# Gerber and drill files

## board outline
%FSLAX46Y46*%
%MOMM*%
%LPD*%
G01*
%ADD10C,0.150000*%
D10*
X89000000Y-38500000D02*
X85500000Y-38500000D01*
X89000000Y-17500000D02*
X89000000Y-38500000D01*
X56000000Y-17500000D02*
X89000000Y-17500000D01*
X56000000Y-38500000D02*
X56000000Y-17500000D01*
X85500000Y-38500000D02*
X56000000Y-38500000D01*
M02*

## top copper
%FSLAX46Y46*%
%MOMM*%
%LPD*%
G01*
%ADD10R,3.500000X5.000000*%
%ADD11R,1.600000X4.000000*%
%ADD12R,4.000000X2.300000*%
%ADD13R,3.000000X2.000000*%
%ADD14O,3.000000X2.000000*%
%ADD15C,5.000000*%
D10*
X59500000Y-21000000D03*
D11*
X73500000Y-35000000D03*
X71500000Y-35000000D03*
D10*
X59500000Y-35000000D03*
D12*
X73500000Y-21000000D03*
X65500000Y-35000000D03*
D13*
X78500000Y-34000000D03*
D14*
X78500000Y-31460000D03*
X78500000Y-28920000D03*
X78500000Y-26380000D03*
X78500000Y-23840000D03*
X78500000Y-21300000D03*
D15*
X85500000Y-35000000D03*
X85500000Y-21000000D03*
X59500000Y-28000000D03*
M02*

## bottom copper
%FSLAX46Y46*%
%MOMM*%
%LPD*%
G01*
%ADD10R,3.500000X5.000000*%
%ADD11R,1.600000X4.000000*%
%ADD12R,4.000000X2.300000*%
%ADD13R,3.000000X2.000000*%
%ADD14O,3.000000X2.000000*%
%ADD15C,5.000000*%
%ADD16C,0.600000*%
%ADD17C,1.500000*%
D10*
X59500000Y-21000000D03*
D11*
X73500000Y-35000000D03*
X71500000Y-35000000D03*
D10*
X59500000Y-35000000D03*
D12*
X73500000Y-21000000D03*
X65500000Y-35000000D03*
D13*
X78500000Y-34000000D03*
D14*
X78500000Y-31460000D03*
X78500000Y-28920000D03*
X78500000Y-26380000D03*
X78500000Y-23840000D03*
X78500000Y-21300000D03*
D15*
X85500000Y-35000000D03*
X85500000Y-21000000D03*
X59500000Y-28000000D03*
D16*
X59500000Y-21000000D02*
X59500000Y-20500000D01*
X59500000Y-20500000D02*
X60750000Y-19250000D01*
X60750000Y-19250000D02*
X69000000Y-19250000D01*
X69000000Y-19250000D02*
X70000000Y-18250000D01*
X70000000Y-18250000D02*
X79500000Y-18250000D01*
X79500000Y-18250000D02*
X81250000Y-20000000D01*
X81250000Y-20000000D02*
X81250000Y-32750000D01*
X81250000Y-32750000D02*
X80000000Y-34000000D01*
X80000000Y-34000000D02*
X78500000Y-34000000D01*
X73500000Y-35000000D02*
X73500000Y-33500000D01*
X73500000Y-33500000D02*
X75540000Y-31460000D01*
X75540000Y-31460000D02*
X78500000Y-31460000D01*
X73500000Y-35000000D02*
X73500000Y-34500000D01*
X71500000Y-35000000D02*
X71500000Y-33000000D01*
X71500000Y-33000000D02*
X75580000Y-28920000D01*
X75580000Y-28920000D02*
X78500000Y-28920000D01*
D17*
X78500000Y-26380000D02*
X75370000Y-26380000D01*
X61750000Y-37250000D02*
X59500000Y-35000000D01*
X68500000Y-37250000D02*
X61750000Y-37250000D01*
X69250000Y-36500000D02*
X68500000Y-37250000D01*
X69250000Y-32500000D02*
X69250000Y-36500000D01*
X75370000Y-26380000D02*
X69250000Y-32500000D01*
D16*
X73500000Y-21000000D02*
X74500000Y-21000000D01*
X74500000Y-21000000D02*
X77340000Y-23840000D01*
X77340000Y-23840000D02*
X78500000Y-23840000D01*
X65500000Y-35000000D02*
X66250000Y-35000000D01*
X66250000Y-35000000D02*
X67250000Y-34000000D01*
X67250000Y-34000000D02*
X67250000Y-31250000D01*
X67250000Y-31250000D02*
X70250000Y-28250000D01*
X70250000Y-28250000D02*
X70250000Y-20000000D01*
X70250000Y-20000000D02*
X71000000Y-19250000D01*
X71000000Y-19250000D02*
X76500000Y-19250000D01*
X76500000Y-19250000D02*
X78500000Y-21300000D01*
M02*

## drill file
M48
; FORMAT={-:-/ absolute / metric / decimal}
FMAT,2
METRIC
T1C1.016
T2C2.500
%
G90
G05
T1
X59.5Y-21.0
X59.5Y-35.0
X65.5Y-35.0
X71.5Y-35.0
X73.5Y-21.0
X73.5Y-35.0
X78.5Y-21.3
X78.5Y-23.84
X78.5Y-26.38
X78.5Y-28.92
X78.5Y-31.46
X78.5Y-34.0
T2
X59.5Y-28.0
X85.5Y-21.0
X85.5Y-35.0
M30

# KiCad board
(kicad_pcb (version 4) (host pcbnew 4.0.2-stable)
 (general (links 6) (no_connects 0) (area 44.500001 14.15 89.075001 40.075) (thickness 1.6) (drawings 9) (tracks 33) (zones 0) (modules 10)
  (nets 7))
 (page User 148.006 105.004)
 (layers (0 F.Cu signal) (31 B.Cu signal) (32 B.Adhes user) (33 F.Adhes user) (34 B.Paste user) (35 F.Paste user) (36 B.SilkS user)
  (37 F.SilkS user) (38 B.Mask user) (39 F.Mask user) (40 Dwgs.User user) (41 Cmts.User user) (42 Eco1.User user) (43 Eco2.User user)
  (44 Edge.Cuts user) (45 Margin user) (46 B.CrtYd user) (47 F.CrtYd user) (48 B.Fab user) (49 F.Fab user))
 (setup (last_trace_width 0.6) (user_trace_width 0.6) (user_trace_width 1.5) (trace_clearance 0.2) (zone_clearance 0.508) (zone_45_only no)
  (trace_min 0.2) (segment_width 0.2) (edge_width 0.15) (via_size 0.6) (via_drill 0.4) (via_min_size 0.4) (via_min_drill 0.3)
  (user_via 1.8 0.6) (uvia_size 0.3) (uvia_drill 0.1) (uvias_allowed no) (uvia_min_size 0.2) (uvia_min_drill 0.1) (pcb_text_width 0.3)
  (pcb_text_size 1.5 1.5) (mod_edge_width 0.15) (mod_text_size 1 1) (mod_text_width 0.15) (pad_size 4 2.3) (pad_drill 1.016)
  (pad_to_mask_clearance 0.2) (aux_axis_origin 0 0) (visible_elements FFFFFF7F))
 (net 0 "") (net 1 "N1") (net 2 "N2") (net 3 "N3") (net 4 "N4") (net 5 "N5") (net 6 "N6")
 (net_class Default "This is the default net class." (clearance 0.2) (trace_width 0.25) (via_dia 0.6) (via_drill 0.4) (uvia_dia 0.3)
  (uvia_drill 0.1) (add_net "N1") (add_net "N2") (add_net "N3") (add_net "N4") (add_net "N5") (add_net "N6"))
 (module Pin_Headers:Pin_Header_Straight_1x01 (layer F.Cu) (at 59.5 21)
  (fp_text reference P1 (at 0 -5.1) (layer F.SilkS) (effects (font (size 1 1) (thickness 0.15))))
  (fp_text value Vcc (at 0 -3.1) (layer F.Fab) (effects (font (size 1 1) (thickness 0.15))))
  (pad 1 thru_hole rect (at 0 0) (size 3.5 5) (drill 1.016) (layers *.Cu *.Mask F.SilkS) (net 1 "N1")))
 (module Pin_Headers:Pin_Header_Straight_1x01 (layer F.Cu) (at 73.5 35)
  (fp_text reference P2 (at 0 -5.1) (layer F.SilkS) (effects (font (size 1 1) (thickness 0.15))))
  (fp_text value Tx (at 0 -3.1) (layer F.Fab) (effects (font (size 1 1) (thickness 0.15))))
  (pad 1 thru_hole rect (at 0 0) (size 1.6 4) (drill 1.016) (layers *.Cu *.Mask F.SilkS) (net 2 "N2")))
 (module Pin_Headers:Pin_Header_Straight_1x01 (layer F.Cu) (at 71.5 35)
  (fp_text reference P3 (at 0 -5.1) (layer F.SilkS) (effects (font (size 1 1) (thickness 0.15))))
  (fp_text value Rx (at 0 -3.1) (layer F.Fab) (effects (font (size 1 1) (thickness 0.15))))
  (pad 1 thru_hole rect (at 0 0) (size 1.6 4) (drill 1.016) (layers *.Cu *.Mask F.SilkS) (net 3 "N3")))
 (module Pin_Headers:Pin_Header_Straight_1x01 (layer F.Cu) (at 59.5 35)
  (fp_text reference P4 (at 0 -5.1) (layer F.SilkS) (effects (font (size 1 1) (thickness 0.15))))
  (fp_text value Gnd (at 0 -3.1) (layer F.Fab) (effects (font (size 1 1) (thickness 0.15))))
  (pad 1 thru_hole rect (at 0 0) (size 3.5 5) (drill 1.016) (layers *.Cu *.Mask F.SilkS) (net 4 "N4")))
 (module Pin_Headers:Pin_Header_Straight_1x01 (layer F.Cu) (at 73.5 21)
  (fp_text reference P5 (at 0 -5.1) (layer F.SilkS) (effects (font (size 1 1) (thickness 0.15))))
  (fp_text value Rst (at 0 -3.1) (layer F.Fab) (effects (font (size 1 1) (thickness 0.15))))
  (pad 1 thru_hole rect (at 0 0) (size 4 2.3) (drill 1.016) (layers *.Cu *.Mask F.SilkS) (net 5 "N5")))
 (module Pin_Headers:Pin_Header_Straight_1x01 (layer F.Cu) (at 65.5 35)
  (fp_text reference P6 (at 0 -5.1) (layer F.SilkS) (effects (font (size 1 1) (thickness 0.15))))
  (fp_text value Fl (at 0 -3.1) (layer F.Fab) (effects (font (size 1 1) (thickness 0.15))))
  (pad 1 thru_hole rect (at 0 0) (size 4 2.3) (drill 1.016) (layers *.Cu *.Mask F.SilkS) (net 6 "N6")))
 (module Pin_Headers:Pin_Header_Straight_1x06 (layer F.Cu) (at 78.5 34 180)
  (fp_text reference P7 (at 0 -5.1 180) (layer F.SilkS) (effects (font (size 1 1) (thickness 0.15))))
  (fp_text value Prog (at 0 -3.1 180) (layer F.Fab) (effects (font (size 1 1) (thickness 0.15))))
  (pad 1 thru_hole rect (at 0 0 180) (size 3 2) (drill 1.016) (layers *.Cu *.Mask F.SilkS) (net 1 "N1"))
  (pad 2 thru_hole oval (at 0 2.54 180) (size 3 2) (drill 1.016) (layers *.Cu *.Mask F.SilkS) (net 2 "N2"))
  (pad 3 thru_hole oval (at 0 5.08 180) (size 3 2) (drill 1.016) (layers *.Cu *.Mask F.SilkS) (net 3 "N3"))
  (pad 4 thru_hole oval (at 0 7.62 180) (size 3 2) (drill 1.016) (layers *.Cu *.Mask F.SilkS) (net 4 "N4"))
  (pad 5 thru_hole oval (at 0 10.16 180) (size 3 2) (drill 1.016) (layers *.Cu *.Mask F.SilkS) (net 5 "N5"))
  (pad 6 thru_hole oval (at 0 12.7 180) (size 3 2) (drill 1.016) (layers *.Cu *.Mask F.SilkS) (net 6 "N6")))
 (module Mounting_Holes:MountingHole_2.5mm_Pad (layer F.Cu) (at 85.5 35)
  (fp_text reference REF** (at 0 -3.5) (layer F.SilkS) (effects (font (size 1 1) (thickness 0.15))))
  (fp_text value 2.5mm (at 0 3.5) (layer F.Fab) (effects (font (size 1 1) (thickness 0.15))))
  (pad 1 thru_hole circle (at 0 0) (size 5 5) (drill 2.5) (layers *.Cu *.Mask F.SilkS)))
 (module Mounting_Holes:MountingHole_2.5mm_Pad (layer F.Cu) (at 85.5 21)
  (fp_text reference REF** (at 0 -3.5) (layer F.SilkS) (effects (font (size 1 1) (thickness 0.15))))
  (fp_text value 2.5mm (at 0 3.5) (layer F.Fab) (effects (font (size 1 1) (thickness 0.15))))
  (pad 1 thru_hole circle (at 0 0) (size 5 5) (drill 2.5) (layers *.Cu *.Mask F.SilkS)))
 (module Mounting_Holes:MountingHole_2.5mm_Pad (layer F.Cu) (at 59.5 28 90)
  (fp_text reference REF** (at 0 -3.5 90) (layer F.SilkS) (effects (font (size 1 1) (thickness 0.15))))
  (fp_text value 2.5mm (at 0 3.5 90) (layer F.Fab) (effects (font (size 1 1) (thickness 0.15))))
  (pad 1 thru_hole circle (at 0 0 90) (size 5 5) (drill 2.5) (layers *.Cu *.Mask F.SilkS)))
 (gr_line (start 89 38.5) (end 85.5 38.5) (angle 90) (layer Edge.Cuts) (width 0.15))
 (gr_line (start 89 17.5) (end 89 38.5) (angle 90) (layer Edge.Cuts) (width 0.15))
 (gr_line (start 56 17.5) (end 89 17.5) (angle 90) (layer Edge.Cuts) (width 0.15))
 (gr_line (start 56 38.5) (end 56 17.5) (angle 90) (layer Edge.Cuts) (width 0.15))
 (gr_line (start 85.5 38.5) (end 56 38.5) (angle 90) (layer Edge.Cuts) (width 0.15))
 (segment (start 59.5 21) (end 59.5 20.5) (width 0.6) (layer B.Cu) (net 1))
 (segment (start 59.5 20.5) (end 60.75 19.25) (width 0.6) (layer B.Cu) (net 1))
 (segment (start 60.75 19.25) (end 69 19.25) (width 0.6) (layer B.Cu) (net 1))
 (segment (start 69 19.25) (end 70 18.25) (width 0.6) (layer B.Cu) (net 1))
 (segment (start 70 18.25) (end 79.5 18.25) (width 0.6) (layer B.Cu) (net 1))
 (segment (start 79.5 18.25) (end 81.25 20) (width 0.6) (layer B.Cu) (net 1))
 (segment (start 81.25 20) (end 81.25 32.75) (width 0.6) (layer B.Cu) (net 1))
 (segment (start 81.25 32.75) (end 80 34) (width 0.6) (layer B.Cu) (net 1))
 (segment (start 80 34) (end 78.5 34) (width 0.6) (layer B.Cu) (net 1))
 (segment (start 73.5 35) (end 73.5 33.5) (width 0.6) (layer B.Cu) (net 2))
 (segment (start 73.5 33.5) (end 75.54 31.46) (width 0.6) (layer B.Cu) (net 2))
 (segment (start 75.54 31.46) (end 78.5 31.46) (width 0.6) (layer B.Cu) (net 2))
 (segment (start 73.5 35) (end 73.5 34.5) (width 0.6) (layer B.Cu) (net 2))
 (segment (start 71.5 35) (end 71.5 33) (width 0.6) (layer B.Cu) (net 3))
 (segment (start 71.5 33) (end 75.58 28.92) (width 0.6) (layer B.Cu) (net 3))
 (segment (start 75.58 28.92) (end 78.5 28.92) (width 0.6) (layer B.Cu) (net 3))
 (segment (start 78.5 26.38) (end 75.37 26.38) (width 1.5) (layer B.Cu) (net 4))
 (segment (start 61.75 37.25) (end 59.5 35) (width 1.5) (layer B.Cu) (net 4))
 (segment (start 68.5 37.25) (end 61.75 37.25) (width 1.5) (layer B.Cu) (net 4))
 (segment (start 69.25 36.5) (end 68.5 37.25) (width 1.5) (layer B.Cu) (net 4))
 (segment (start 69.25 32.5) (end 69.25 36.5) (width 1.5) (layer B.Cu) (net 4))
 (segment (start 75.37 26.38) (end 69.25 32.5) (width 1.5) (layer B.Cu) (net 4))
 (segment (start 73.5 21) (end 74.5 21) (width 0.6) (layer B.Cu) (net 5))
 (segment (start 74.5 21) (end 77.34 23.84) (width 0.6) (layer B.Cu) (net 5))
 (segment (start 77.34 23.84) (end 78.5 23.84) (width 0.6) (layer B.Cu) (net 5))
 (segment (start 65.5 35) (end 66.25 35) (width 0.6) (layer B.Cu) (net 6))
 (segment (start 66.25 35) (end 67.25 34) (width 0.6) (layer B.Cu) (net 6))
 (segment (start 67.25 34) (end 67.25 31.25) (width 0.6) (layer B.Cu) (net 6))
 (segment (start 67.25 31.25) (end 70.25 28.25) (width 0.6) (layer B.Cu) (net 6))
 (segment (start 70.25 28.25) (end 70.25 20) (width 0.6) (layer B.Cu) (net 6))
 (segment (start 70.25 20) (end 71 19.25) (width 0.6) (layer B.Cu) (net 6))
 (segment (start 71 19.25) (end 76.5 19.25) (width 0.6) (layer B.Cu) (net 6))
 (segment (start 76.5 19.25) (end 78.5 21.3) (width 0.6) (layer B.Cu) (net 6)))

